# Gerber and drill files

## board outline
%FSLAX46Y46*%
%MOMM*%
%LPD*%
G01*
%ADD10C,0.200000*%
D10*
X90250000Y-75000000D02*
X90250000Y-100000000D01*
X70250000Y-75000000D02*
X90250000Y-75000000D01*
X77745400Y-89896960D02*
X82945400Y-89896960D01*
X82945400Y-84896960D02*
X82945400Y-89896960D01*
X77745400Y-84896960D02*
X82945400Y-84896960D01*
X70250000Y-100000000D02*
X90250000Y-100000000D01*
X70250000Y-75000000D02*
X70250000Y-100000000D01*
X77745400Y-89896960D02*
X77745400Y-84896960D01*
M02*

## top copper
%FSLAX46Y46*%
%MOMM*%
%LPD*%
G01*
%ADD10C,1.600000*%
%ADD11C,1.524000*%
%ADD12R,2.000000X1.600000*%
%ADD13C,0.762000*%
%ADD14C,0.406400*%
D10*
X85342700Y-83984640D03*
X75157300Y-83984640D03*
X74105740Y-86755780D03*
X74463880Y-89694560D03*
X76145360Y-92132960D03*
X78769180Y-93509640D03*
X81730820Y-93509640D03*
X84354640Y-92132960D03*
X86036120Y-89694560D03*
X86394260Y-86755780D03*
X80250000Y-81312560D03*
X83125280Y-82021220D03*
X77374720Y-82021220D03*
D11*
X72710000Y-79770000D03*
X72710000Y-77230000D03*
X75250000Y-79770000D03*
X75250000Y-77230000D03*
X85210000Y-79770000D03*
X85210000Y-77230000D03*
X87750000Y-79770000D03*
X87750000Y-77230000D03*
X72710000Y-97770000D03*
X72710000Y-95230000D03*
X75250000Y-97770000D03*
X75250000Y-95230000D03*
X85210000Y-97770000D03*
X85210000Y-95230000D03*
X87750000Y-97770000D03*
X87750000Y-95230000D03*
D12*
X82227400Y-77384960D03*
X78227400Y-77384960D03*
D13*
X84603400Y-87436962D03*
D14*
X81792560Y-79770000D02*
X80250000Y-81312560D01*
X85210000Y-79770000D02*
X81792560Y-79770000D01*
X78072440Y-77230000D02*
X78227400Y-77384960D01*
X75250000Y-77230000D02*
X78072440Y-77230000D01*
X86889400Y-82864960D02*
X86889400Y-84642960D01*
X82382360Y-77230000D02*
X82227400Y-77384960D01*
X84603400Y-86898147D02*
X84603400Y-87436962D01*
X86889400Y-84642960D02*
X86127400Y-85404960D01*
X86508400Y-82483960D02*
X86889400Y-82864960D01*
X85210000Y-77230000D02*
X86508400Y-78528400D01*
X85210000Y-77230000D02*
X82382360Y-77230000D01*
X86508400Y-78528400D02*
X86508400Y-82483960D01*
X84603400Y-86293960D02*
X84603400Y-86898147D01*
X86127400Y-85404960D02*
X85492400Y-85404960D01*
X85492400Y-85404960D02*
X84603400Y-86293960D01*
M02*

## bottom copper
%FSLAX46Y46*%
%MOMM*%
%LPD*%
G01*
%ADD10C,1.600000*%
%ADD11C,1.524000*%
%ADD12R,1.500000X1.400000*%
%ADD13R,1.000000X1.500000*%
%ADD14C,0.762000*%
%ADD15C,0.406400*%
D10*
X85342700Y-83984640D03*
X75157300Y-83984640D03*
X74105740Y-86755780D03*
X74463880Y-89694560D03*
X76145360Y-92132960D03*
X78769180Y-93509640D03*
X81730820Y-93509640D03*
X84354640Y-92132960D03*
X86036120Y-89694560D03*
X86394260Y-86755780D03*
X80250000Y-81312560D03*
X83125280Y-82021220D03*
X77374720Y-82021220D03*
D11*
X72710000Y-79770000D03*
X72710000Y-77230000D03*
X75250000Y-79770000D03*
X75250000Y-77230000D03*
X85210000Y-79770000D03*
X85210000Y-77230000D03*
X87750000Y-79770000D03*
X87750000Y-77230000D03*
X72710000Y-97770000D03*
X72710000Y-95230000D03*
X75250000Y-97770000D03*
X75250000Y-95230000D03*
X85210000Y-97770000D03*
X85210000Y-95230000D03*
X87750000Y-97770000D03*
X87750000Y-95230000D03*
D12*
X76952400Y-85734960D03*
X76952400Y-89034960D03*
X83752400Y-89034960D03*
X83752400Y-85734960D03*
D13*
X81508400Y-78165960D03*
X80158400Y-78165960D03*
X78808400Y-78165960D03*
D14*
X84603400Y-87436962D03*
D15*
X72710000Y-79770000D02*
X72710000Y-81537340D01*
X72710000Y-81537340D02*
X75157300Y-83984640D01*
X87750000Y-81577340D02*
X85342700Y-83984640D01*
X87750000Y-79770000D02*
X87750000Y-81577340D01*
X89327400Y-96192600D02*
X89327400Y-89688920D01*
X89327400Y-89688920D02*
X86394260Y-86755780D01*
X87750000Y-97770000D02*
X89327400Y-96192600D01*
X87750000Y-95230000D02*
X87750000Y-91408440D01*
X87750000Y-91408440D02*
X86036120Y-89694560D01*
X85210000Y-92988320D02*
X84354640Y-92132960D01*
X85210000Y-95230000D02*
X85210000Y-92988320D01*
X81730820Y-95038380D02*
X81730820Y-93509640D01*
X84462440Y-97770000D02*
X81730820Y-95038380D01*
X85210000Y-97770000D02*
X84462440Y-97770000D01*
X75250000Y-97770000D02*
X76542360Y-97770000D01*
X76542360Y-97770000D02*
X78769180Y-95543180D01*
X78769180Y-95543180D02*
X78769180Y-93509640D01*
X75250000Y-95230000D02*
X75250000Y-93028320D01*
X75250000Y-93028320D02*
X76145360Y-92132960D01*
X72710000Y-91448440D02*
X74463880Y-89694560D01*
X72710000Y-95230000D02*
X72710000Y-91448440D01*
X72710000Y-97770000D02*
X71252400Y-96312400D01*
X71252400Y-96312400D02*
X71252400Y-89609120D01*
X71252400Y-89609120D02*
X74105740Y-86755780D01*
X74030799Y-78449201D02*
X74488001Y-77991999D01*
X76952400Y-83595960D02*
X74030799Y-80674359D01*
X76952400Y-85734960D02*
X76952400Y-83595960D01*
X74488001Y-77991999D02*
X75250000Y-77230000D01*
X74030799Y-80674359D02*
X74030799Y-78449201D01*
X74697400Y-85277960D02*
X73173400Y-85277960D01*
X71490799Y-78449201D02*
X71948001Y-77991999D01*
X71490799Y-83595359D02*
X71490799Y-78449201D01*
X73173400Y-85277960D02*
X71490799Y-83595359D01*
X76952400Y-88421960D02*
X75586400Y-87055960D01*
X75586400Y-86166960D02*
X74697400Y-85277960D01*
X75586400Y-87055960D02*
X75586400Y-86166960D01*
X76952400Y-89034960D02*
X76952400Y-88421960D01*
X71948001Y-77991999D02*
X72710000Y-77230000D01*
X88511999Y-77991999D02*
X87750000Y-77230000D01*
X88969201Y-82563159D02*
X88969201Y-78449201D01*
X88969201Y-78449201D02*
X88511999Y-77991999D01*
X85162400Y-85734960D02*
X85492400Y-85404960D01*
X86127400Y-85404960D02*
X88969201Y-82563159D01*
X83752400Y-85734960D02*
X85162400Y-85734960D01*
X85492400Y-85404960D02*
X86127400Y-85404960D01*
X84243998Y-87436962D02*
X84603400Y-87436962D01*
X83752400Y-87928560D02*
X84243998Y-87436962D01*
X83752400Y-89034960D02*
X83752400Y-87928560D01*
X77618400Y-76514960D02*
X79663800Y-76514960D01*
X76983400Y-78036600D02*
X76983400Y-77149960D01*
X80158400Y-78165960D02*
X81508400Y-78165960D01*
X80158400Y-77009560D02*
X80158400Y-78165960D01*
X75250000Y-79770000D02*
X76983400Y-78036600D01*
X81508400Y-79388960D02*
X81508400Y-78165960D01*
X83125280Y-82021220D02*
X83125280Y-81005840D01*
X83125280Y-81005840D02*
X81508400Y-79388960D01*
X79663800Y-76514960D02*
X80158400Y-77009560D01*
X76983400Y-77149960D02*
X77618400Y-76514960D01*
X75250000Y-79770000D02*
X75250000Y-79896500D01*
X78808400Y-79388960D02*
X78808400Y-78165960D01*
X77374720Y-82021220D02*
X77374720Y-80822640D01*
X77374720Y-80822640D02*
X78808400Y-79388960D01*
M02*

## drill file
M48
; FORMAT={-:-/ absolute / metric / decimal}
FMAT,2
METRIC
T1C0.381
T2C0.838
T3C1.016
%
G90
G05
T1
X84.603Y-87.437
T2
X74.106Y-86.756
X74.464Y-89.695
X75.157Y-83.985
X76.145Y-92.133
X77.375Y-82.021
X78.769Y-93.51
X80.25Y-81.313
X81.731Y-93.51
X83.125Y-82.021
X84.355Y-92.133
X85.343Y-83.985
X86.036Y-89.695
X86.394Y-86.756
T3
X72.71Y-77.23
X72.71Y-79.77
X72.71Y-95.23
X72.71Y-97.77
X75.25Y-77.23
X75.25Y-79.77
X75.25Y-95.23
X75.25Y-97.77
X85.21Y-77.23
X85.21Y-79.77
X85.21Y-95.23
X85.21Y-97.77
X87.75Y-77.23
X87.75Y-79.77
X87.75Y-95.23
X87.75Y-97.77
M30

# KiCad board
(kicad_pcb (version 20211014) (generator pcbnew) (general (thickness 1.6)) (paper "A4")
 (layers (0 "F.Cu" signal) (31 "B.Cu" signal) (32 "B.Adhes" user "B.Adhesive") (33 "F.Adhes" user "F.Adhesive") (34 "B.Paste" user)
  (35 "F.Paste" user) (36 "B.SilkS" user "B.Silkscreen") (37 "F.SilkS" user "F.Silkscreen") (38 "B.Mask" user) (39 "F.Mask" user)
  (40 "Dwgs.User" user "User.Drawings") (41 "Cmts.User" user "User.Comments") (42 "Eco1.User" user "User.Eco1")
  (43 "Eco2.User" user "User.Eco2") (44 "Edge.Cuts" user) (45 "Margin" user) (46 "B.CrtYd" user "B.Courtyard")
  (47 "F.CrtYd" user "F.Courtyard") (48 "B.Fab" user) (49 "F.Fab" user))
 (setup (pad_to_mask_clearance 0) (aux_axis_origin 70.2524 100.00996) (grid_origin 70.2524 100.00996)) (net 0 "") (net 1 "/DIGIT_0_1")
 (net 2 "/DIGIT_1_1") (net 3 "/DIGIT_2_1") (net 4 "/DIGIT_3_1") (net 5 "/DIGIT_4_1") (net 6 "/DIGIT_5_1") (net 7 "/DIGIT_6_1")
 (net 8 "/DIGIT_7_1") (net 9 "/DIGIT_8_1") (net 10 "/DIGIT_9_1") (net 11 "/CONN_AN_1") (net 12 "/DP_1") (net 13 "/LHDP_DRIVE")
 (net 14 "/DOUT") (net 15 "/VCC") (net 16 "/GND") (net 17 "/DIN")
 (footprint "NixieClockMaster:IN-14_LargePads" (layer "F.Cu") (at 80.25 87.5 180)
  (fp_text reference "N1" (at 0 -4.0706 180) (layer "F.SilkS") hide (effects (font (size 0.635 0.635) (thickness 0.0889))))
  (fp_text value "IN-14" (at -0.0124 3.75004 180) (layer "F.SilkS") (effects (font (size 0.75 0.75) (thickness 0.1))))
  (pad "0" thru_hole circle locked (at -5.0927 3.51536 180) (size 1.6 1.6) (drill 0.8382) (layers *.Cu *.Mask "F.Paste" "F.SilkS")
   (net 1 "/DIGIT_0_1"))
  (pad "1" thru_hole circle locked (at 5.0927 3.51536 180) (size 1.6 1.6) (drill 0.8382) (layers *.Cu *.Mask "F.Paste" "F.SilkS")
   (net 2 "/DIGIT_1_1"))
  (pad "2" thru_hole circle locked (at 6.14426 0.74422 180) (size 1.6 1.6) (drill 0.8382) (layers *.Cu *.Mask "F.Paste" "F.SilkS")
   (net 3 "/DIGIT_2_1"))
  (pad "3" thru_hole circle locked (at 5.78612 -2.19456 180) (size 1.6 1.6) (drill 0.8382) (layers *.Cu *.Mask "F.Paste" "F.SilkS")
   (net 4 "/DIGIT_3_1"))
  (pad "4" thru_hole circle locked (at 4.10464 -4.63296 180) (size 1.6 1.6) (drill 0.8382) (layers *.Cu *.Mask "F.Paste" "F.SilkS")
   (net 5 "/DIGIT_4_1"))
  (pad "5" thru_hole circle locked (at 1.48082 -6.00964 180) (size 1.6 1.6) (drill 0.8382) (layers *.Cu *.Mask "F.Paste" "F.SilkS")
   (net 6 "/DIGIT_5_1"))
  (pad "6" thru_hole circle locked (at -1.48082 -6.00964 180) (size 1.6 1.6) (drill 0.8382) (layers *.Cu *.Mask "F.Paste" "F.SilkS")
   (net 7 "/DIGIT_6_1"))
  (pad "7" thru_hole circle locked (at -4.10464 -4.63296 180) (size 1.6 1.6) (drill 0.8382) (layers *.Cu *.Mask "F.Paste" "F.SilkS")
   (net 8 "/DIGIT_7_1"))
  (pad "8" thru_hole circle locked (at -5.78612 -2.19456 180) (size 1.6 1.6) (drill 0.8382) (layers *.Cu *.Mask "F.Paste" "F.SilkS")
   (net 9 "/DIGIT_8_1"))
  (pad "9" thru_hole circle locked (at -6.14426 0.74422 180) (size 1.6 1.6) (drill 0.8382) (layers *.Cu *.Mask "F.Paste" "F.SilkS")
   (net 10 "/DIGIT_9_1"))
  (pad "A" thru_hole circle locked (at 0 6.18744 180) (size 1.6 1.6) (drill 0.8382) (layers *.Cu *.Mask "F.Paste" "F.SilkS")
   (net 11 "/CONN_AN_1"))
  (pad "LHDP" thru_hole circle locked (at -2.87528 5.47878 180) (size 1.6 1.6) (drill 0.8382) (layers *.Cu *.Mask "F.Paste" "F.SilkS")
   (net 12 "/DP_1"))
  (pad "RHDP" thru_hole circle locked (at 2.87528 5.47878 180) (size 1.6 1.6) (drill 0.8382) (layers *.Cu *.Mask "F.Paste" "F.SilkS")
   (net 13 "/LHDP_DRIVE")))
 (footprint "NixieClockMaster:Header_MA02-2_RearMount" (layer "F.Cu") (at 75.25 78.5)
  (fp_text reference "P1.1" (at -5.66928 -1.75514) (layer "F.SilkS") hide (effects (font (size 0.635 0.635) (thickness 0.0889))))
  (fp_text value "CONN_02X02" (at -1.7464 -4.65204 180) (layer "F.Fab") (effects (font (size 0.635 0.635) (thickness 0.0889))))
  (pad "1" thru_hole circle locked (at -2.54 1.27) (size 1.524 1.524) (drill 1.016) (layers *.Cu *.Mask "F.Paste" "F.SilkS")
   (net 2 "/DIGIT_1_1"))
  (pad "2" thru_hole circle locked (at -2.54 -1.27) (size 1.524 1.524) (drill 1.016) (layers *.Cu *.Mask "F.Paste" "F.SilkS")
   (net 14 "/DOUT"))
  (pad "3" thru_hole circle locked (at 0 1.27) (size 1.524 1.524) (drill 1.016) (layers *.Cu *.Mask "F.Paste" "F.SilkS") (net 12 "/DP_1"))
  (pad "4" thru_hole circle locked (at 0 -1.27) (size 1.524 1.524) (drill 1.016) (layers *.Cu *.Mask "F.Paste" "F.SilkS") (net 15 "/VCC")))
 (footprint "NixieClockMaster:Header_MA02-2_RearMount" (layer "F.Cu") (at 87.75 78.5)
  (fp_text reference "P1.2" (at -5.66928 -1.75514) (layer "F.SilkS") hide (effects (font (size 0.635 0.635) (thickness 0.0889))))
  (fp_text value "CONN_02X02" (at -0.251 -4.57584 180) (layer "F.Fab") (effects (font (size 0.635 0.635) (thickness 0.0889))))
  (pad "1" thru_hole circle locked (at -2.54 1.27) (size 1.524 1.524) (drill 1.016) (layers *.Cu *.Mask "F.Paste" "F.SilkS")
   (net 11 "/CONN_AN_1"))
  (pad "2" thru_hole circle locked (at -2.54 -1.27) (size 1.524 1.524) (drill 1.016) (layers *.Cu *.Mask "F.Paste" "F.SilkS")
   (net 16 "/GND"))
  (pad "3" thru_hole circle locked (at 0 1.27) (size 1.524 1.524) (drill 1.016) (layers *.Cu *.Mask "F.Paste" "F.SilkS")
   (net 1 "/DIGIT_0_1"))
  (pad "4" thru_hole circle locked (at 0 -1.27) (size 1.524 1.524) (drill 1.016) (layers *.Cu *.Mask "F.Paste" "F.SilkS") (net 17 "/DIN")))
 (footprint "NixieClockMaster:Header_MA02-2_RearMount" (layer "F.Cu") (at 75.25 96.5)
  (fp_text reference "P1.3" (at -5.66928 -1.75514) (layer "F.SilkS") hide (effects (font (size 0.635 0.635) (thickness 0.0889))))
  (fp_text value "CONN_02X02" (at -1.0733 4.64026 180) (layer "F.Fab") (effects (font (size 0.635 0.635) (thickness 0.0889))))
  (pad "1" thru_hole circle locked (at -2.54 1.27) (size 1.524 1.524) (drill 1.016) (layers *.Cu *.Mask "F.Paste" "F.SilkS")
   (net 3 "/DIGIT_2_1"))
  (pad "2" thru_hole circle locked (at -2.54 -1.27) (size 1.524 1.524) (drill 1.016) (layers *.Cu *.Mask "F.Paste" "F.SilkS")
   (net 4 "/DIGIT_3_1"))
  (pad "3" thru_hole circle locked (at 0 1.27) (size 1.524 1.524) (drill 1.016) (layers *.Cu *.Mask "F.Paste" "F.SilkS")
   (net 6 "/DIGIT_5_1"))
  (pad "4" thru_hole circle locked (at 0 -1.27) (size 1.524 1.524) (drill 1.016) (layers *.Cu *.Mask "F.Paste" "F.SilkS")
   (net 5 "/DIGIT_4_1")))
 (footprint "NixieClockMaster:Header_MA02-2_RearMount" (layer "F.Cu") (at 87.75 96.5)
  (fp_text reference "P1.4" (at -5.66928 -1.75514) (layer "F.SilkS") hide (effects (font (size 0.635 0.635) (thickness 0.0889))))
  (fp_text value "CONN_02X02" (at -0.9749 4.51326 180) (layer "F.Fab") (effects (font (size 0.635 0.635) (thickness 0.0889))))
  (pad "1" thru_hole circle locked (at -2.54 1.27) (size 1.524 1.524) (drill 1.016) (layers *.Cu *.Mask "F.Paste" "F.SilkS")
   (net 7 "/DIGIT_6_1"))
  (pad "2" thru_hole circle locked (at -2.54 -1.27) (size 1.524 1.524) (drill 1.016) (layers *.Cu *.Mask "F.Paste" "F.SilkS")
   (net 8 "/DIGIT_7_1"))
  (pad "3" thru_hole circle locked (at 0 1.27) (size 1.524 1.524) (drill 1.016) (layers *.Cu *.Mask "F.Paste" "F.SilkS")
   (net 10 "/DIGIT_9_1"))
  (pad "4" thru_hole circle locked (at 0 -1.27) (size 1.524 1.524) (drill 1.016) (layers *.Cu *.Mask "F.Paste" "F.SilkS")
   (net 9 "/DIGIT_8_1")))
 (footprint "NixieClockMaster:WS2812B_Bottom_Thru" (layer "F.Cu") (at 80.3524 87.38496 90)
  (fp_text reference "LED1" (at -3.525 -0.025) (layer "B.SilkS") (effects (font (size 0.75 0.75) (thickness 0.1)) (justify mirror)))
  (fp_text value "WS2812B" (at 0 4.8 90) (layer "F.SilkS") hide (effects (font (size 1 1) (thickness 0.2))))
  (pad "1" smd rect locked (at 1.65 -3.4 90) (size 1.4 1.5) (layers "B.Cu" "B.Paste" "B.Mask") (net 15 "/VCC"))
  (pad "2" smd rect locked (at -1.65 -3.4 90) (size 1.4 1.5) (layers "B.Cu" "B.Paste" "B.Mask") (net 14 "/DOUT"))
  (pad "3" smd rect locked (at -1.65 3.4 90) (size 1.4 1.5) (layers "B.Cu" "B.Paste" "B.Mask") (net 16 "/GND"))
  (pad "4" smd rect locked (at 1.65 3.4 90) (size 1.4 1.5) (layers "B.Cu" "B.Paste" "B.Mask") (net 17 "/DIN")))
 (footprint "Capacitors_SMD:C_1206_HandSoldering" (layer "F.Cu") (at 80.2274 77.38496 180)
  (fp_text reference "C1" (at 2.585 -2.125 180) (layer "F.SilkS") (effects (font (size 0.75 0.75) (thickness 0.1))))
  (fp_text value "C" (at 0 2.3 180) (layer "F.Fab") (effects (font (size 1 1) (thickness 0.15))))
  (pad "1" smd rect locked (at -2 0 180) (size 2 1.6) (layers "F.Cu" "F.Paste" "F.Mask") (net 16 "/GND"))
  (pad "2" smd rect locked (at 2 0 180) (size 2 1.6) (layers "F.Cu" "F.Paste" "F.Mask") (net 15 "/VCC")))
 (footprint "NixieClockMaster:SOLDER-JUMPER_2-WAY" (layer "B.Cu") (at 80.1584 78.16596 180)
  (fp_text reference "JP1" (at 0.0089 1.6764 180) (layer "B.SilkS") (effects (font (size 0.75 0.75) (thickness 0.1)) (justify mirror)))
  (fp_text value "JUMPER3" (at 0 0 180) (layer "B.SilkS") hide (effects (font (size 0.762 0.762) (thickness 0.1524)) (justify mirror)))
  (pad "1" smd rect locked (at -1.35 0 180) (size 1 1.5) (layers "B.Cu" "B.Paste" "B.Mask") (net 12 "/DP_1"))
  (pad "2" smd rect locked (at 0 0 180) (size 1 1.5) (layers "B.Cu" "B.Paste" "B.Mask") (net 12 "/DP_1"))
  (pad "3" smd rect locked (at 1.35 0 180) (size 1 1.5) (layers "B.Cu" "B.Paste" "B.Mask") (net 13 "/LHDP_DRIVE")))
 (gr_line (start 90.25 75) (end 90.25 100) (layer "Edge.Cuts") (width 0.2))
 (gr_line (start 70.25 75) (end 90.25 75) (layer "Edge.Cuts") (width 0.2))
 (gr_line (start 77.7454 89.89696) (end 82.9454 89.89696) (layer "Edge.Cuts") (width 0.2))
 (gr_line (start 82.9454 84.89696) (end 82.9454 89.89696) (layer "Edge.Cuts") (width 0.2))
 (gr_line (start 77.7454 84.89696) (end 82.9454 84.89696) (layer "Edge.Cuts") (width 0.2))
 (gr_line (start 70.25 100) (end 90.25 100) (layer "Edge.Cuts") (width 0.2))
 (gr_line (start 70.25 75) (end 70.25 100) (layer "Edge.Cuts") (width 0.2))
 (gr_line (start 77.7454 89.89696) (end 77.7454 84.89696) (layer "Edge.Cuts") (width 0.2))
 (segment (start 72.71 79.77) (end 72.71 81.53734) (width 0.4064) (layer "B.Cu") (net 2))
 (segment (start 72.71 81.53734) (end 75.1573 83.98464) (width 0.4064) (layer "B.Cu") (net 2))
 (segment (start 87.75 81.57734) (end 85.3427 83.98464) (width 0.4064) (layer "B.Cu") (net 1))
 (segment (start 87.75 79.77) (end 87.75 81.57734) (width 0.4064) (layer "B.Cu") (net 1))
 (segment (start 89.3274 96.1926) (end 89.3274 89.68892) (width 0.4064) (layer "B.Cu") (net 10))
 (segment (start 89.3274 89.68892) (end 86.39426 86.75578) (width 0.4064) (layer "B.Cu") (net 10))
 (segment (start 87.75 97.77) (end 89.3274 96.1926) (width 0.4064) (layer "B.Cu") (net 10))
 (segment (start 87.75 95.23) (end 87.75 91.40844) (width 0.4064) (layer "B.Cu") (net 9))
 (segment (start 87.75 91.40844) (end 86.03612 89.69456) (width 0.4064) (layer "B.Cu") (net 9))
 (segment (start 85.21 92.98832) (end 84.35464 92.13296) (width 0.4064) (layer "B.Cu") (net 8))
 (segment (start 85.21 95.23) (end 85.21 92.98832) (width 0.4064) (layer "B.Cu") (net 8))
 (segment (start 81.73082 95.03838) (end 81.73082 93.50964) (width 0.4064) (layer "B.Cu") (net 7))
 (segment (start 84.46244 97.77) (end 81.73082 95.03838) (width 0.4064) (layer "B.Cu") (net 7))
 (segment (start 85.21 97.77) (end 84.46244 97.77) (width 0.4064) (layer "B.Cu") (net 7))
 (segment (start 75.25 97.77) (end 76.54236 97.77) (width 0.4064) (layer "B.Cu") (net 6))
 (segment (start 76.54236 97.77) (end 78.76918 95.54318) (width 0.4064) (layer "B.Cu") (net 6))
 (segment (start 78.76918 95.54318) (end 78.76918 93.50964) (width 0.4064) (layer "B.Cu") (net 6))
 (segment (start 75.25 95.23) (end 75.25 93.02832) (width 0.4064) (layer "B.Cu") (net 5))
 (segment (start 75.25 93.02832) (end 76.14536 92.13296) (width 0.4064) (layer "B.Cu") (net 5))
 (segment (start 72.71 91.44844) (end 74.46388 89.69456) (width 0.4064) (layer "B.Cu") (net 4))
 (segment (start 72.71 95.23) (end 72.71 91.44844) (width 0.4064) (layer "B.Cu") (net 4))
 (segment (start 72.71 97.77) (end 71.2524 96.3124) (width 0.4064) (layer "B.Cu") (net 3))
 (segment (start 71.2524 96.3124) (end 71.2524 89.60912) (width 0.4064) (layer "B.Cu") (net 3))
 (segment (start 71.2524 89.60912) (end 74.10574 86.75578) (width 0.4064) (layer "B.Cu") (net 3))
 (segment (start 81.79256 79.77) (end 80.25 81.31256) (width 0.4064) (layer "F.Cu") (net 11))
 (segment (start 85.21 79.77) (end 81.79256 79.77) (width 0.4064) (layer "F.Cu") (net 11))
 (segment (start 78.07244 77.23) (end 78.2274 77.38496) (width 0.4064) (layer "F.Cu") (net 15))
 (segment (start 75.25 77.23) (end 78.07244 77.23) (width 0.4064) (layer "F.Cu") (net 15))
 (segment (start 74.030799 78.449201) (end 74.488001 77.991999) (width 0.4064) (layer "B.Cu") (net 15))
 (segment (start 76.9524 83.59596) (end 74.030799 80.674359) (width 0.4064) (layer "B.Cu") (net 15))
 (segment (start 76.9524 85.73496) (end 76.9524 83.59596) (width 0.4064) (layer "B.Cu") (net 15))
 (segment (start 74.488001 77.991999) (end 75.25 77.23) (width 0.4064) (layer "B.Cu") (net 15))
 (segment (start 74.030799 80.674359) (end 74.030799 78.449201) (width 0.4064) (layer "B.Cu") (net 15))
 (segment (start 74.6974 85.27796) (end 73.1734 85.27796) (width 0.4064) (layer "B.Cu") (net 14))
 (segment (start 71.490799 78.449201) (end 71.948001 77.991999) (width 0.4064) (layer "B.Cu") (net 14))
 (segment (start 71.490799 83.595359) (end 71.490799 78.449201) (width 0.4064) (layer "B.Cu") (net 14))
 (segment (start 73.1734 85.27796) (end 71.490799 83.595359) (width 0.4064) (layer "B.Cu") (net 14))
 (segment (start 76.9524 88.42196) (end 75.5864 87.05596) (width 0.4064) (layer "B.Cu") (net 14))
 (segment (start 75.5864 86.16696) (end 74.6974 85.27796) (width 0.4064) (layer "B.Cu") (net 14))
 (segment (start 75.5864 87.05596) (end 75.5864 86.16696) (width 0.4064) (layer "B.Cu") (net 14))
 (segment (start 76.9524 89.03496) (end 76.9524 88.42196) (width 0.4064) (layer "B.Cu") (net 14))
 (segment (start 71.948001 77.991999) (end 72.71 77.23) (width 0.4064) (layer "B.Cu") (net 14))
 (segment (start 88.511999 77.991999) (end 87.75 77.23) (width 0.4064) (layer "B.Cu") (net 17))
 (segment (start 88.969201 82.563159) (end 88.969201 78.449201) (width 0.4064) (layer "B.Cu") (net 17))
 (segment (start 88.969201 78.449201) (end 88.511999 77.991999) (width 0.4064) (layer "B.Cu") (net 17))
 (segment (start 85.1624 85.73496) (end 85.4924 85.40496) (width 0.4064) (layer "B.Cu") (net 17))
 (segment (start 86.1274 85.40496) (end 88.969201 82.563159) (width 0.4064) (layer "B.Cu") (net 17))
 (segment (start 83.7524 85.73496) (end 85.1624 85.73496) (width 0.4064) (layer "B.Cu") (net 17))
 (segment (start 85.4924 85.40496) (end 86.1274 85.40496) (width 0.4064) (layer "B.Cu") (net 17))
 (segment (start 86.8894 82.86496) (end 86.8894 84.64296) (width 0.4064) (layer "F.Cu") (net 16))
 (segment (start 82.38236 77.23) (end 82.2274 77.38496) (width 0.4064) (layer "F.Cu") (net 16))
 (segment (start 84.6034 86.898147) (end 84.6034 87.436962) (width 0.4064) (layer "F.Cu") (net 16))
 (segment (start 86.8894 84.64296) (end 86.1274 85.40496) (width 0.4064) (layer "F.Cu") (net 16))
 (segment (start 86.5084 82.48396) (end 86.8894 82.86496) (width 0.4064) (layer "F.Cu") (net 16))
 (segment (start 85.21 77.23) (end 86.5084 78.5284) (width 0.4064) (layer "F.Cu") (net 16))
 (segment (start 85.21 77.23) (end 82.38236 77.23) (width 0.4064) (layer "F.Cu") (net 16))
 (segment (start 86.5084 78.5284) (end 86.5084 82.48396) (width 0.4064) (layer "F.Cu") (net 16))
 (segment (start 84.6034 86.29396) (end 84.6034 86.898147) (width 0.4064) (layer "F.Cu") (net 16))
 (segment (start 86.1274 85.40496) (end 85.4924 85.40496) (width 0.4064) (layer "F.Cu") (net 16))
 (segment (start 85.4924 85.40496) (end 84.6034 86.29396) (width 0.4064) (layer "F.Cu") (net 16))
 (via (at 84.6034 87.436962) (size 0.762) (drill 0.381) (layers "F.Cu" "B.Cu") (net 16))
 (segment (start 84.243998 87.436962) (end 84.6034 87.436962) (width 0.4064) (layer "B.Cu") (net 16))
 (segment (start 83.7524 87.92856) (end 84.243998 87.436962) (width 0.4064) (layer "B.Cu") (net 16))
 (segment (start 83.7524 89.03496) (end 83.7524 87.92856) (width 0.4064) (layer "B.Cu") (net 16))
 (segment (start 77.6184 76.51496) (end 79.6638 76.51496) (width 0.4064) (layer "B.Cu") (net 12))
 (segment (start 76.9834 78.0366) (end 76.9834 77.14996) (width 0.4064) (layer "B.Cu") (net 12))
 (segment (start 80.1584 78.16596) (end 81.5084 78.16596) (width 0.4064) (layer "B.Cu") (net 12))
 (segment (start 80.1584 77.00956) (end 80.1584 78.16596) (width 0.4064) (layer "B.Cu") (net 12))
 (segment (start 75.25 79.77) (end 76.9834 78.0366) (width 0.4064) (layer "B.Cu") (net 12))
 (segment (start 81.5084 79.38896) (end 81.5084 78.16596) (width 0.4064) (layer "B.Cu") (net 12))
 (segment (start 83.12528 82.02122) (end 83.12528 81.00584) (width 0.4064) (layer "B.Cu") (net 12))
 (segment (start 83.12528 81.00584) (end 81.5084 79.38896) (width 0.4064) (layer "B.Cu") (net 12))
 (segment (start 79.6638 76.51496) (end 80.1584 77.00956) (width 0.4064) (layer "B.Cu") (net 12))
 (segment (start 76.9834 77.14996) (end 77.6184 76.51496) (width 0.4064) (layer "B.Cu") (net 12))
 (segment (start 75.25 79.77) (end 75.25 79.8965) (width 0.4064) (layer "B.Cu") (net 12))
 (segment (start 78.8084 79.38896) (end 78.8084 78.16596) (width 0.4064) (layer "B.Cu") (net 13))
 (segment (start 77.37472 82.02122) (end 77.37472 80.82264) (width 0.4064) (layer "B.Cu") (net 13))
 (segment (start 77.37472 80.82264) (end 78.8084 79.38896) (width 0.4064) (layer "B.Cu") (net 13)))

